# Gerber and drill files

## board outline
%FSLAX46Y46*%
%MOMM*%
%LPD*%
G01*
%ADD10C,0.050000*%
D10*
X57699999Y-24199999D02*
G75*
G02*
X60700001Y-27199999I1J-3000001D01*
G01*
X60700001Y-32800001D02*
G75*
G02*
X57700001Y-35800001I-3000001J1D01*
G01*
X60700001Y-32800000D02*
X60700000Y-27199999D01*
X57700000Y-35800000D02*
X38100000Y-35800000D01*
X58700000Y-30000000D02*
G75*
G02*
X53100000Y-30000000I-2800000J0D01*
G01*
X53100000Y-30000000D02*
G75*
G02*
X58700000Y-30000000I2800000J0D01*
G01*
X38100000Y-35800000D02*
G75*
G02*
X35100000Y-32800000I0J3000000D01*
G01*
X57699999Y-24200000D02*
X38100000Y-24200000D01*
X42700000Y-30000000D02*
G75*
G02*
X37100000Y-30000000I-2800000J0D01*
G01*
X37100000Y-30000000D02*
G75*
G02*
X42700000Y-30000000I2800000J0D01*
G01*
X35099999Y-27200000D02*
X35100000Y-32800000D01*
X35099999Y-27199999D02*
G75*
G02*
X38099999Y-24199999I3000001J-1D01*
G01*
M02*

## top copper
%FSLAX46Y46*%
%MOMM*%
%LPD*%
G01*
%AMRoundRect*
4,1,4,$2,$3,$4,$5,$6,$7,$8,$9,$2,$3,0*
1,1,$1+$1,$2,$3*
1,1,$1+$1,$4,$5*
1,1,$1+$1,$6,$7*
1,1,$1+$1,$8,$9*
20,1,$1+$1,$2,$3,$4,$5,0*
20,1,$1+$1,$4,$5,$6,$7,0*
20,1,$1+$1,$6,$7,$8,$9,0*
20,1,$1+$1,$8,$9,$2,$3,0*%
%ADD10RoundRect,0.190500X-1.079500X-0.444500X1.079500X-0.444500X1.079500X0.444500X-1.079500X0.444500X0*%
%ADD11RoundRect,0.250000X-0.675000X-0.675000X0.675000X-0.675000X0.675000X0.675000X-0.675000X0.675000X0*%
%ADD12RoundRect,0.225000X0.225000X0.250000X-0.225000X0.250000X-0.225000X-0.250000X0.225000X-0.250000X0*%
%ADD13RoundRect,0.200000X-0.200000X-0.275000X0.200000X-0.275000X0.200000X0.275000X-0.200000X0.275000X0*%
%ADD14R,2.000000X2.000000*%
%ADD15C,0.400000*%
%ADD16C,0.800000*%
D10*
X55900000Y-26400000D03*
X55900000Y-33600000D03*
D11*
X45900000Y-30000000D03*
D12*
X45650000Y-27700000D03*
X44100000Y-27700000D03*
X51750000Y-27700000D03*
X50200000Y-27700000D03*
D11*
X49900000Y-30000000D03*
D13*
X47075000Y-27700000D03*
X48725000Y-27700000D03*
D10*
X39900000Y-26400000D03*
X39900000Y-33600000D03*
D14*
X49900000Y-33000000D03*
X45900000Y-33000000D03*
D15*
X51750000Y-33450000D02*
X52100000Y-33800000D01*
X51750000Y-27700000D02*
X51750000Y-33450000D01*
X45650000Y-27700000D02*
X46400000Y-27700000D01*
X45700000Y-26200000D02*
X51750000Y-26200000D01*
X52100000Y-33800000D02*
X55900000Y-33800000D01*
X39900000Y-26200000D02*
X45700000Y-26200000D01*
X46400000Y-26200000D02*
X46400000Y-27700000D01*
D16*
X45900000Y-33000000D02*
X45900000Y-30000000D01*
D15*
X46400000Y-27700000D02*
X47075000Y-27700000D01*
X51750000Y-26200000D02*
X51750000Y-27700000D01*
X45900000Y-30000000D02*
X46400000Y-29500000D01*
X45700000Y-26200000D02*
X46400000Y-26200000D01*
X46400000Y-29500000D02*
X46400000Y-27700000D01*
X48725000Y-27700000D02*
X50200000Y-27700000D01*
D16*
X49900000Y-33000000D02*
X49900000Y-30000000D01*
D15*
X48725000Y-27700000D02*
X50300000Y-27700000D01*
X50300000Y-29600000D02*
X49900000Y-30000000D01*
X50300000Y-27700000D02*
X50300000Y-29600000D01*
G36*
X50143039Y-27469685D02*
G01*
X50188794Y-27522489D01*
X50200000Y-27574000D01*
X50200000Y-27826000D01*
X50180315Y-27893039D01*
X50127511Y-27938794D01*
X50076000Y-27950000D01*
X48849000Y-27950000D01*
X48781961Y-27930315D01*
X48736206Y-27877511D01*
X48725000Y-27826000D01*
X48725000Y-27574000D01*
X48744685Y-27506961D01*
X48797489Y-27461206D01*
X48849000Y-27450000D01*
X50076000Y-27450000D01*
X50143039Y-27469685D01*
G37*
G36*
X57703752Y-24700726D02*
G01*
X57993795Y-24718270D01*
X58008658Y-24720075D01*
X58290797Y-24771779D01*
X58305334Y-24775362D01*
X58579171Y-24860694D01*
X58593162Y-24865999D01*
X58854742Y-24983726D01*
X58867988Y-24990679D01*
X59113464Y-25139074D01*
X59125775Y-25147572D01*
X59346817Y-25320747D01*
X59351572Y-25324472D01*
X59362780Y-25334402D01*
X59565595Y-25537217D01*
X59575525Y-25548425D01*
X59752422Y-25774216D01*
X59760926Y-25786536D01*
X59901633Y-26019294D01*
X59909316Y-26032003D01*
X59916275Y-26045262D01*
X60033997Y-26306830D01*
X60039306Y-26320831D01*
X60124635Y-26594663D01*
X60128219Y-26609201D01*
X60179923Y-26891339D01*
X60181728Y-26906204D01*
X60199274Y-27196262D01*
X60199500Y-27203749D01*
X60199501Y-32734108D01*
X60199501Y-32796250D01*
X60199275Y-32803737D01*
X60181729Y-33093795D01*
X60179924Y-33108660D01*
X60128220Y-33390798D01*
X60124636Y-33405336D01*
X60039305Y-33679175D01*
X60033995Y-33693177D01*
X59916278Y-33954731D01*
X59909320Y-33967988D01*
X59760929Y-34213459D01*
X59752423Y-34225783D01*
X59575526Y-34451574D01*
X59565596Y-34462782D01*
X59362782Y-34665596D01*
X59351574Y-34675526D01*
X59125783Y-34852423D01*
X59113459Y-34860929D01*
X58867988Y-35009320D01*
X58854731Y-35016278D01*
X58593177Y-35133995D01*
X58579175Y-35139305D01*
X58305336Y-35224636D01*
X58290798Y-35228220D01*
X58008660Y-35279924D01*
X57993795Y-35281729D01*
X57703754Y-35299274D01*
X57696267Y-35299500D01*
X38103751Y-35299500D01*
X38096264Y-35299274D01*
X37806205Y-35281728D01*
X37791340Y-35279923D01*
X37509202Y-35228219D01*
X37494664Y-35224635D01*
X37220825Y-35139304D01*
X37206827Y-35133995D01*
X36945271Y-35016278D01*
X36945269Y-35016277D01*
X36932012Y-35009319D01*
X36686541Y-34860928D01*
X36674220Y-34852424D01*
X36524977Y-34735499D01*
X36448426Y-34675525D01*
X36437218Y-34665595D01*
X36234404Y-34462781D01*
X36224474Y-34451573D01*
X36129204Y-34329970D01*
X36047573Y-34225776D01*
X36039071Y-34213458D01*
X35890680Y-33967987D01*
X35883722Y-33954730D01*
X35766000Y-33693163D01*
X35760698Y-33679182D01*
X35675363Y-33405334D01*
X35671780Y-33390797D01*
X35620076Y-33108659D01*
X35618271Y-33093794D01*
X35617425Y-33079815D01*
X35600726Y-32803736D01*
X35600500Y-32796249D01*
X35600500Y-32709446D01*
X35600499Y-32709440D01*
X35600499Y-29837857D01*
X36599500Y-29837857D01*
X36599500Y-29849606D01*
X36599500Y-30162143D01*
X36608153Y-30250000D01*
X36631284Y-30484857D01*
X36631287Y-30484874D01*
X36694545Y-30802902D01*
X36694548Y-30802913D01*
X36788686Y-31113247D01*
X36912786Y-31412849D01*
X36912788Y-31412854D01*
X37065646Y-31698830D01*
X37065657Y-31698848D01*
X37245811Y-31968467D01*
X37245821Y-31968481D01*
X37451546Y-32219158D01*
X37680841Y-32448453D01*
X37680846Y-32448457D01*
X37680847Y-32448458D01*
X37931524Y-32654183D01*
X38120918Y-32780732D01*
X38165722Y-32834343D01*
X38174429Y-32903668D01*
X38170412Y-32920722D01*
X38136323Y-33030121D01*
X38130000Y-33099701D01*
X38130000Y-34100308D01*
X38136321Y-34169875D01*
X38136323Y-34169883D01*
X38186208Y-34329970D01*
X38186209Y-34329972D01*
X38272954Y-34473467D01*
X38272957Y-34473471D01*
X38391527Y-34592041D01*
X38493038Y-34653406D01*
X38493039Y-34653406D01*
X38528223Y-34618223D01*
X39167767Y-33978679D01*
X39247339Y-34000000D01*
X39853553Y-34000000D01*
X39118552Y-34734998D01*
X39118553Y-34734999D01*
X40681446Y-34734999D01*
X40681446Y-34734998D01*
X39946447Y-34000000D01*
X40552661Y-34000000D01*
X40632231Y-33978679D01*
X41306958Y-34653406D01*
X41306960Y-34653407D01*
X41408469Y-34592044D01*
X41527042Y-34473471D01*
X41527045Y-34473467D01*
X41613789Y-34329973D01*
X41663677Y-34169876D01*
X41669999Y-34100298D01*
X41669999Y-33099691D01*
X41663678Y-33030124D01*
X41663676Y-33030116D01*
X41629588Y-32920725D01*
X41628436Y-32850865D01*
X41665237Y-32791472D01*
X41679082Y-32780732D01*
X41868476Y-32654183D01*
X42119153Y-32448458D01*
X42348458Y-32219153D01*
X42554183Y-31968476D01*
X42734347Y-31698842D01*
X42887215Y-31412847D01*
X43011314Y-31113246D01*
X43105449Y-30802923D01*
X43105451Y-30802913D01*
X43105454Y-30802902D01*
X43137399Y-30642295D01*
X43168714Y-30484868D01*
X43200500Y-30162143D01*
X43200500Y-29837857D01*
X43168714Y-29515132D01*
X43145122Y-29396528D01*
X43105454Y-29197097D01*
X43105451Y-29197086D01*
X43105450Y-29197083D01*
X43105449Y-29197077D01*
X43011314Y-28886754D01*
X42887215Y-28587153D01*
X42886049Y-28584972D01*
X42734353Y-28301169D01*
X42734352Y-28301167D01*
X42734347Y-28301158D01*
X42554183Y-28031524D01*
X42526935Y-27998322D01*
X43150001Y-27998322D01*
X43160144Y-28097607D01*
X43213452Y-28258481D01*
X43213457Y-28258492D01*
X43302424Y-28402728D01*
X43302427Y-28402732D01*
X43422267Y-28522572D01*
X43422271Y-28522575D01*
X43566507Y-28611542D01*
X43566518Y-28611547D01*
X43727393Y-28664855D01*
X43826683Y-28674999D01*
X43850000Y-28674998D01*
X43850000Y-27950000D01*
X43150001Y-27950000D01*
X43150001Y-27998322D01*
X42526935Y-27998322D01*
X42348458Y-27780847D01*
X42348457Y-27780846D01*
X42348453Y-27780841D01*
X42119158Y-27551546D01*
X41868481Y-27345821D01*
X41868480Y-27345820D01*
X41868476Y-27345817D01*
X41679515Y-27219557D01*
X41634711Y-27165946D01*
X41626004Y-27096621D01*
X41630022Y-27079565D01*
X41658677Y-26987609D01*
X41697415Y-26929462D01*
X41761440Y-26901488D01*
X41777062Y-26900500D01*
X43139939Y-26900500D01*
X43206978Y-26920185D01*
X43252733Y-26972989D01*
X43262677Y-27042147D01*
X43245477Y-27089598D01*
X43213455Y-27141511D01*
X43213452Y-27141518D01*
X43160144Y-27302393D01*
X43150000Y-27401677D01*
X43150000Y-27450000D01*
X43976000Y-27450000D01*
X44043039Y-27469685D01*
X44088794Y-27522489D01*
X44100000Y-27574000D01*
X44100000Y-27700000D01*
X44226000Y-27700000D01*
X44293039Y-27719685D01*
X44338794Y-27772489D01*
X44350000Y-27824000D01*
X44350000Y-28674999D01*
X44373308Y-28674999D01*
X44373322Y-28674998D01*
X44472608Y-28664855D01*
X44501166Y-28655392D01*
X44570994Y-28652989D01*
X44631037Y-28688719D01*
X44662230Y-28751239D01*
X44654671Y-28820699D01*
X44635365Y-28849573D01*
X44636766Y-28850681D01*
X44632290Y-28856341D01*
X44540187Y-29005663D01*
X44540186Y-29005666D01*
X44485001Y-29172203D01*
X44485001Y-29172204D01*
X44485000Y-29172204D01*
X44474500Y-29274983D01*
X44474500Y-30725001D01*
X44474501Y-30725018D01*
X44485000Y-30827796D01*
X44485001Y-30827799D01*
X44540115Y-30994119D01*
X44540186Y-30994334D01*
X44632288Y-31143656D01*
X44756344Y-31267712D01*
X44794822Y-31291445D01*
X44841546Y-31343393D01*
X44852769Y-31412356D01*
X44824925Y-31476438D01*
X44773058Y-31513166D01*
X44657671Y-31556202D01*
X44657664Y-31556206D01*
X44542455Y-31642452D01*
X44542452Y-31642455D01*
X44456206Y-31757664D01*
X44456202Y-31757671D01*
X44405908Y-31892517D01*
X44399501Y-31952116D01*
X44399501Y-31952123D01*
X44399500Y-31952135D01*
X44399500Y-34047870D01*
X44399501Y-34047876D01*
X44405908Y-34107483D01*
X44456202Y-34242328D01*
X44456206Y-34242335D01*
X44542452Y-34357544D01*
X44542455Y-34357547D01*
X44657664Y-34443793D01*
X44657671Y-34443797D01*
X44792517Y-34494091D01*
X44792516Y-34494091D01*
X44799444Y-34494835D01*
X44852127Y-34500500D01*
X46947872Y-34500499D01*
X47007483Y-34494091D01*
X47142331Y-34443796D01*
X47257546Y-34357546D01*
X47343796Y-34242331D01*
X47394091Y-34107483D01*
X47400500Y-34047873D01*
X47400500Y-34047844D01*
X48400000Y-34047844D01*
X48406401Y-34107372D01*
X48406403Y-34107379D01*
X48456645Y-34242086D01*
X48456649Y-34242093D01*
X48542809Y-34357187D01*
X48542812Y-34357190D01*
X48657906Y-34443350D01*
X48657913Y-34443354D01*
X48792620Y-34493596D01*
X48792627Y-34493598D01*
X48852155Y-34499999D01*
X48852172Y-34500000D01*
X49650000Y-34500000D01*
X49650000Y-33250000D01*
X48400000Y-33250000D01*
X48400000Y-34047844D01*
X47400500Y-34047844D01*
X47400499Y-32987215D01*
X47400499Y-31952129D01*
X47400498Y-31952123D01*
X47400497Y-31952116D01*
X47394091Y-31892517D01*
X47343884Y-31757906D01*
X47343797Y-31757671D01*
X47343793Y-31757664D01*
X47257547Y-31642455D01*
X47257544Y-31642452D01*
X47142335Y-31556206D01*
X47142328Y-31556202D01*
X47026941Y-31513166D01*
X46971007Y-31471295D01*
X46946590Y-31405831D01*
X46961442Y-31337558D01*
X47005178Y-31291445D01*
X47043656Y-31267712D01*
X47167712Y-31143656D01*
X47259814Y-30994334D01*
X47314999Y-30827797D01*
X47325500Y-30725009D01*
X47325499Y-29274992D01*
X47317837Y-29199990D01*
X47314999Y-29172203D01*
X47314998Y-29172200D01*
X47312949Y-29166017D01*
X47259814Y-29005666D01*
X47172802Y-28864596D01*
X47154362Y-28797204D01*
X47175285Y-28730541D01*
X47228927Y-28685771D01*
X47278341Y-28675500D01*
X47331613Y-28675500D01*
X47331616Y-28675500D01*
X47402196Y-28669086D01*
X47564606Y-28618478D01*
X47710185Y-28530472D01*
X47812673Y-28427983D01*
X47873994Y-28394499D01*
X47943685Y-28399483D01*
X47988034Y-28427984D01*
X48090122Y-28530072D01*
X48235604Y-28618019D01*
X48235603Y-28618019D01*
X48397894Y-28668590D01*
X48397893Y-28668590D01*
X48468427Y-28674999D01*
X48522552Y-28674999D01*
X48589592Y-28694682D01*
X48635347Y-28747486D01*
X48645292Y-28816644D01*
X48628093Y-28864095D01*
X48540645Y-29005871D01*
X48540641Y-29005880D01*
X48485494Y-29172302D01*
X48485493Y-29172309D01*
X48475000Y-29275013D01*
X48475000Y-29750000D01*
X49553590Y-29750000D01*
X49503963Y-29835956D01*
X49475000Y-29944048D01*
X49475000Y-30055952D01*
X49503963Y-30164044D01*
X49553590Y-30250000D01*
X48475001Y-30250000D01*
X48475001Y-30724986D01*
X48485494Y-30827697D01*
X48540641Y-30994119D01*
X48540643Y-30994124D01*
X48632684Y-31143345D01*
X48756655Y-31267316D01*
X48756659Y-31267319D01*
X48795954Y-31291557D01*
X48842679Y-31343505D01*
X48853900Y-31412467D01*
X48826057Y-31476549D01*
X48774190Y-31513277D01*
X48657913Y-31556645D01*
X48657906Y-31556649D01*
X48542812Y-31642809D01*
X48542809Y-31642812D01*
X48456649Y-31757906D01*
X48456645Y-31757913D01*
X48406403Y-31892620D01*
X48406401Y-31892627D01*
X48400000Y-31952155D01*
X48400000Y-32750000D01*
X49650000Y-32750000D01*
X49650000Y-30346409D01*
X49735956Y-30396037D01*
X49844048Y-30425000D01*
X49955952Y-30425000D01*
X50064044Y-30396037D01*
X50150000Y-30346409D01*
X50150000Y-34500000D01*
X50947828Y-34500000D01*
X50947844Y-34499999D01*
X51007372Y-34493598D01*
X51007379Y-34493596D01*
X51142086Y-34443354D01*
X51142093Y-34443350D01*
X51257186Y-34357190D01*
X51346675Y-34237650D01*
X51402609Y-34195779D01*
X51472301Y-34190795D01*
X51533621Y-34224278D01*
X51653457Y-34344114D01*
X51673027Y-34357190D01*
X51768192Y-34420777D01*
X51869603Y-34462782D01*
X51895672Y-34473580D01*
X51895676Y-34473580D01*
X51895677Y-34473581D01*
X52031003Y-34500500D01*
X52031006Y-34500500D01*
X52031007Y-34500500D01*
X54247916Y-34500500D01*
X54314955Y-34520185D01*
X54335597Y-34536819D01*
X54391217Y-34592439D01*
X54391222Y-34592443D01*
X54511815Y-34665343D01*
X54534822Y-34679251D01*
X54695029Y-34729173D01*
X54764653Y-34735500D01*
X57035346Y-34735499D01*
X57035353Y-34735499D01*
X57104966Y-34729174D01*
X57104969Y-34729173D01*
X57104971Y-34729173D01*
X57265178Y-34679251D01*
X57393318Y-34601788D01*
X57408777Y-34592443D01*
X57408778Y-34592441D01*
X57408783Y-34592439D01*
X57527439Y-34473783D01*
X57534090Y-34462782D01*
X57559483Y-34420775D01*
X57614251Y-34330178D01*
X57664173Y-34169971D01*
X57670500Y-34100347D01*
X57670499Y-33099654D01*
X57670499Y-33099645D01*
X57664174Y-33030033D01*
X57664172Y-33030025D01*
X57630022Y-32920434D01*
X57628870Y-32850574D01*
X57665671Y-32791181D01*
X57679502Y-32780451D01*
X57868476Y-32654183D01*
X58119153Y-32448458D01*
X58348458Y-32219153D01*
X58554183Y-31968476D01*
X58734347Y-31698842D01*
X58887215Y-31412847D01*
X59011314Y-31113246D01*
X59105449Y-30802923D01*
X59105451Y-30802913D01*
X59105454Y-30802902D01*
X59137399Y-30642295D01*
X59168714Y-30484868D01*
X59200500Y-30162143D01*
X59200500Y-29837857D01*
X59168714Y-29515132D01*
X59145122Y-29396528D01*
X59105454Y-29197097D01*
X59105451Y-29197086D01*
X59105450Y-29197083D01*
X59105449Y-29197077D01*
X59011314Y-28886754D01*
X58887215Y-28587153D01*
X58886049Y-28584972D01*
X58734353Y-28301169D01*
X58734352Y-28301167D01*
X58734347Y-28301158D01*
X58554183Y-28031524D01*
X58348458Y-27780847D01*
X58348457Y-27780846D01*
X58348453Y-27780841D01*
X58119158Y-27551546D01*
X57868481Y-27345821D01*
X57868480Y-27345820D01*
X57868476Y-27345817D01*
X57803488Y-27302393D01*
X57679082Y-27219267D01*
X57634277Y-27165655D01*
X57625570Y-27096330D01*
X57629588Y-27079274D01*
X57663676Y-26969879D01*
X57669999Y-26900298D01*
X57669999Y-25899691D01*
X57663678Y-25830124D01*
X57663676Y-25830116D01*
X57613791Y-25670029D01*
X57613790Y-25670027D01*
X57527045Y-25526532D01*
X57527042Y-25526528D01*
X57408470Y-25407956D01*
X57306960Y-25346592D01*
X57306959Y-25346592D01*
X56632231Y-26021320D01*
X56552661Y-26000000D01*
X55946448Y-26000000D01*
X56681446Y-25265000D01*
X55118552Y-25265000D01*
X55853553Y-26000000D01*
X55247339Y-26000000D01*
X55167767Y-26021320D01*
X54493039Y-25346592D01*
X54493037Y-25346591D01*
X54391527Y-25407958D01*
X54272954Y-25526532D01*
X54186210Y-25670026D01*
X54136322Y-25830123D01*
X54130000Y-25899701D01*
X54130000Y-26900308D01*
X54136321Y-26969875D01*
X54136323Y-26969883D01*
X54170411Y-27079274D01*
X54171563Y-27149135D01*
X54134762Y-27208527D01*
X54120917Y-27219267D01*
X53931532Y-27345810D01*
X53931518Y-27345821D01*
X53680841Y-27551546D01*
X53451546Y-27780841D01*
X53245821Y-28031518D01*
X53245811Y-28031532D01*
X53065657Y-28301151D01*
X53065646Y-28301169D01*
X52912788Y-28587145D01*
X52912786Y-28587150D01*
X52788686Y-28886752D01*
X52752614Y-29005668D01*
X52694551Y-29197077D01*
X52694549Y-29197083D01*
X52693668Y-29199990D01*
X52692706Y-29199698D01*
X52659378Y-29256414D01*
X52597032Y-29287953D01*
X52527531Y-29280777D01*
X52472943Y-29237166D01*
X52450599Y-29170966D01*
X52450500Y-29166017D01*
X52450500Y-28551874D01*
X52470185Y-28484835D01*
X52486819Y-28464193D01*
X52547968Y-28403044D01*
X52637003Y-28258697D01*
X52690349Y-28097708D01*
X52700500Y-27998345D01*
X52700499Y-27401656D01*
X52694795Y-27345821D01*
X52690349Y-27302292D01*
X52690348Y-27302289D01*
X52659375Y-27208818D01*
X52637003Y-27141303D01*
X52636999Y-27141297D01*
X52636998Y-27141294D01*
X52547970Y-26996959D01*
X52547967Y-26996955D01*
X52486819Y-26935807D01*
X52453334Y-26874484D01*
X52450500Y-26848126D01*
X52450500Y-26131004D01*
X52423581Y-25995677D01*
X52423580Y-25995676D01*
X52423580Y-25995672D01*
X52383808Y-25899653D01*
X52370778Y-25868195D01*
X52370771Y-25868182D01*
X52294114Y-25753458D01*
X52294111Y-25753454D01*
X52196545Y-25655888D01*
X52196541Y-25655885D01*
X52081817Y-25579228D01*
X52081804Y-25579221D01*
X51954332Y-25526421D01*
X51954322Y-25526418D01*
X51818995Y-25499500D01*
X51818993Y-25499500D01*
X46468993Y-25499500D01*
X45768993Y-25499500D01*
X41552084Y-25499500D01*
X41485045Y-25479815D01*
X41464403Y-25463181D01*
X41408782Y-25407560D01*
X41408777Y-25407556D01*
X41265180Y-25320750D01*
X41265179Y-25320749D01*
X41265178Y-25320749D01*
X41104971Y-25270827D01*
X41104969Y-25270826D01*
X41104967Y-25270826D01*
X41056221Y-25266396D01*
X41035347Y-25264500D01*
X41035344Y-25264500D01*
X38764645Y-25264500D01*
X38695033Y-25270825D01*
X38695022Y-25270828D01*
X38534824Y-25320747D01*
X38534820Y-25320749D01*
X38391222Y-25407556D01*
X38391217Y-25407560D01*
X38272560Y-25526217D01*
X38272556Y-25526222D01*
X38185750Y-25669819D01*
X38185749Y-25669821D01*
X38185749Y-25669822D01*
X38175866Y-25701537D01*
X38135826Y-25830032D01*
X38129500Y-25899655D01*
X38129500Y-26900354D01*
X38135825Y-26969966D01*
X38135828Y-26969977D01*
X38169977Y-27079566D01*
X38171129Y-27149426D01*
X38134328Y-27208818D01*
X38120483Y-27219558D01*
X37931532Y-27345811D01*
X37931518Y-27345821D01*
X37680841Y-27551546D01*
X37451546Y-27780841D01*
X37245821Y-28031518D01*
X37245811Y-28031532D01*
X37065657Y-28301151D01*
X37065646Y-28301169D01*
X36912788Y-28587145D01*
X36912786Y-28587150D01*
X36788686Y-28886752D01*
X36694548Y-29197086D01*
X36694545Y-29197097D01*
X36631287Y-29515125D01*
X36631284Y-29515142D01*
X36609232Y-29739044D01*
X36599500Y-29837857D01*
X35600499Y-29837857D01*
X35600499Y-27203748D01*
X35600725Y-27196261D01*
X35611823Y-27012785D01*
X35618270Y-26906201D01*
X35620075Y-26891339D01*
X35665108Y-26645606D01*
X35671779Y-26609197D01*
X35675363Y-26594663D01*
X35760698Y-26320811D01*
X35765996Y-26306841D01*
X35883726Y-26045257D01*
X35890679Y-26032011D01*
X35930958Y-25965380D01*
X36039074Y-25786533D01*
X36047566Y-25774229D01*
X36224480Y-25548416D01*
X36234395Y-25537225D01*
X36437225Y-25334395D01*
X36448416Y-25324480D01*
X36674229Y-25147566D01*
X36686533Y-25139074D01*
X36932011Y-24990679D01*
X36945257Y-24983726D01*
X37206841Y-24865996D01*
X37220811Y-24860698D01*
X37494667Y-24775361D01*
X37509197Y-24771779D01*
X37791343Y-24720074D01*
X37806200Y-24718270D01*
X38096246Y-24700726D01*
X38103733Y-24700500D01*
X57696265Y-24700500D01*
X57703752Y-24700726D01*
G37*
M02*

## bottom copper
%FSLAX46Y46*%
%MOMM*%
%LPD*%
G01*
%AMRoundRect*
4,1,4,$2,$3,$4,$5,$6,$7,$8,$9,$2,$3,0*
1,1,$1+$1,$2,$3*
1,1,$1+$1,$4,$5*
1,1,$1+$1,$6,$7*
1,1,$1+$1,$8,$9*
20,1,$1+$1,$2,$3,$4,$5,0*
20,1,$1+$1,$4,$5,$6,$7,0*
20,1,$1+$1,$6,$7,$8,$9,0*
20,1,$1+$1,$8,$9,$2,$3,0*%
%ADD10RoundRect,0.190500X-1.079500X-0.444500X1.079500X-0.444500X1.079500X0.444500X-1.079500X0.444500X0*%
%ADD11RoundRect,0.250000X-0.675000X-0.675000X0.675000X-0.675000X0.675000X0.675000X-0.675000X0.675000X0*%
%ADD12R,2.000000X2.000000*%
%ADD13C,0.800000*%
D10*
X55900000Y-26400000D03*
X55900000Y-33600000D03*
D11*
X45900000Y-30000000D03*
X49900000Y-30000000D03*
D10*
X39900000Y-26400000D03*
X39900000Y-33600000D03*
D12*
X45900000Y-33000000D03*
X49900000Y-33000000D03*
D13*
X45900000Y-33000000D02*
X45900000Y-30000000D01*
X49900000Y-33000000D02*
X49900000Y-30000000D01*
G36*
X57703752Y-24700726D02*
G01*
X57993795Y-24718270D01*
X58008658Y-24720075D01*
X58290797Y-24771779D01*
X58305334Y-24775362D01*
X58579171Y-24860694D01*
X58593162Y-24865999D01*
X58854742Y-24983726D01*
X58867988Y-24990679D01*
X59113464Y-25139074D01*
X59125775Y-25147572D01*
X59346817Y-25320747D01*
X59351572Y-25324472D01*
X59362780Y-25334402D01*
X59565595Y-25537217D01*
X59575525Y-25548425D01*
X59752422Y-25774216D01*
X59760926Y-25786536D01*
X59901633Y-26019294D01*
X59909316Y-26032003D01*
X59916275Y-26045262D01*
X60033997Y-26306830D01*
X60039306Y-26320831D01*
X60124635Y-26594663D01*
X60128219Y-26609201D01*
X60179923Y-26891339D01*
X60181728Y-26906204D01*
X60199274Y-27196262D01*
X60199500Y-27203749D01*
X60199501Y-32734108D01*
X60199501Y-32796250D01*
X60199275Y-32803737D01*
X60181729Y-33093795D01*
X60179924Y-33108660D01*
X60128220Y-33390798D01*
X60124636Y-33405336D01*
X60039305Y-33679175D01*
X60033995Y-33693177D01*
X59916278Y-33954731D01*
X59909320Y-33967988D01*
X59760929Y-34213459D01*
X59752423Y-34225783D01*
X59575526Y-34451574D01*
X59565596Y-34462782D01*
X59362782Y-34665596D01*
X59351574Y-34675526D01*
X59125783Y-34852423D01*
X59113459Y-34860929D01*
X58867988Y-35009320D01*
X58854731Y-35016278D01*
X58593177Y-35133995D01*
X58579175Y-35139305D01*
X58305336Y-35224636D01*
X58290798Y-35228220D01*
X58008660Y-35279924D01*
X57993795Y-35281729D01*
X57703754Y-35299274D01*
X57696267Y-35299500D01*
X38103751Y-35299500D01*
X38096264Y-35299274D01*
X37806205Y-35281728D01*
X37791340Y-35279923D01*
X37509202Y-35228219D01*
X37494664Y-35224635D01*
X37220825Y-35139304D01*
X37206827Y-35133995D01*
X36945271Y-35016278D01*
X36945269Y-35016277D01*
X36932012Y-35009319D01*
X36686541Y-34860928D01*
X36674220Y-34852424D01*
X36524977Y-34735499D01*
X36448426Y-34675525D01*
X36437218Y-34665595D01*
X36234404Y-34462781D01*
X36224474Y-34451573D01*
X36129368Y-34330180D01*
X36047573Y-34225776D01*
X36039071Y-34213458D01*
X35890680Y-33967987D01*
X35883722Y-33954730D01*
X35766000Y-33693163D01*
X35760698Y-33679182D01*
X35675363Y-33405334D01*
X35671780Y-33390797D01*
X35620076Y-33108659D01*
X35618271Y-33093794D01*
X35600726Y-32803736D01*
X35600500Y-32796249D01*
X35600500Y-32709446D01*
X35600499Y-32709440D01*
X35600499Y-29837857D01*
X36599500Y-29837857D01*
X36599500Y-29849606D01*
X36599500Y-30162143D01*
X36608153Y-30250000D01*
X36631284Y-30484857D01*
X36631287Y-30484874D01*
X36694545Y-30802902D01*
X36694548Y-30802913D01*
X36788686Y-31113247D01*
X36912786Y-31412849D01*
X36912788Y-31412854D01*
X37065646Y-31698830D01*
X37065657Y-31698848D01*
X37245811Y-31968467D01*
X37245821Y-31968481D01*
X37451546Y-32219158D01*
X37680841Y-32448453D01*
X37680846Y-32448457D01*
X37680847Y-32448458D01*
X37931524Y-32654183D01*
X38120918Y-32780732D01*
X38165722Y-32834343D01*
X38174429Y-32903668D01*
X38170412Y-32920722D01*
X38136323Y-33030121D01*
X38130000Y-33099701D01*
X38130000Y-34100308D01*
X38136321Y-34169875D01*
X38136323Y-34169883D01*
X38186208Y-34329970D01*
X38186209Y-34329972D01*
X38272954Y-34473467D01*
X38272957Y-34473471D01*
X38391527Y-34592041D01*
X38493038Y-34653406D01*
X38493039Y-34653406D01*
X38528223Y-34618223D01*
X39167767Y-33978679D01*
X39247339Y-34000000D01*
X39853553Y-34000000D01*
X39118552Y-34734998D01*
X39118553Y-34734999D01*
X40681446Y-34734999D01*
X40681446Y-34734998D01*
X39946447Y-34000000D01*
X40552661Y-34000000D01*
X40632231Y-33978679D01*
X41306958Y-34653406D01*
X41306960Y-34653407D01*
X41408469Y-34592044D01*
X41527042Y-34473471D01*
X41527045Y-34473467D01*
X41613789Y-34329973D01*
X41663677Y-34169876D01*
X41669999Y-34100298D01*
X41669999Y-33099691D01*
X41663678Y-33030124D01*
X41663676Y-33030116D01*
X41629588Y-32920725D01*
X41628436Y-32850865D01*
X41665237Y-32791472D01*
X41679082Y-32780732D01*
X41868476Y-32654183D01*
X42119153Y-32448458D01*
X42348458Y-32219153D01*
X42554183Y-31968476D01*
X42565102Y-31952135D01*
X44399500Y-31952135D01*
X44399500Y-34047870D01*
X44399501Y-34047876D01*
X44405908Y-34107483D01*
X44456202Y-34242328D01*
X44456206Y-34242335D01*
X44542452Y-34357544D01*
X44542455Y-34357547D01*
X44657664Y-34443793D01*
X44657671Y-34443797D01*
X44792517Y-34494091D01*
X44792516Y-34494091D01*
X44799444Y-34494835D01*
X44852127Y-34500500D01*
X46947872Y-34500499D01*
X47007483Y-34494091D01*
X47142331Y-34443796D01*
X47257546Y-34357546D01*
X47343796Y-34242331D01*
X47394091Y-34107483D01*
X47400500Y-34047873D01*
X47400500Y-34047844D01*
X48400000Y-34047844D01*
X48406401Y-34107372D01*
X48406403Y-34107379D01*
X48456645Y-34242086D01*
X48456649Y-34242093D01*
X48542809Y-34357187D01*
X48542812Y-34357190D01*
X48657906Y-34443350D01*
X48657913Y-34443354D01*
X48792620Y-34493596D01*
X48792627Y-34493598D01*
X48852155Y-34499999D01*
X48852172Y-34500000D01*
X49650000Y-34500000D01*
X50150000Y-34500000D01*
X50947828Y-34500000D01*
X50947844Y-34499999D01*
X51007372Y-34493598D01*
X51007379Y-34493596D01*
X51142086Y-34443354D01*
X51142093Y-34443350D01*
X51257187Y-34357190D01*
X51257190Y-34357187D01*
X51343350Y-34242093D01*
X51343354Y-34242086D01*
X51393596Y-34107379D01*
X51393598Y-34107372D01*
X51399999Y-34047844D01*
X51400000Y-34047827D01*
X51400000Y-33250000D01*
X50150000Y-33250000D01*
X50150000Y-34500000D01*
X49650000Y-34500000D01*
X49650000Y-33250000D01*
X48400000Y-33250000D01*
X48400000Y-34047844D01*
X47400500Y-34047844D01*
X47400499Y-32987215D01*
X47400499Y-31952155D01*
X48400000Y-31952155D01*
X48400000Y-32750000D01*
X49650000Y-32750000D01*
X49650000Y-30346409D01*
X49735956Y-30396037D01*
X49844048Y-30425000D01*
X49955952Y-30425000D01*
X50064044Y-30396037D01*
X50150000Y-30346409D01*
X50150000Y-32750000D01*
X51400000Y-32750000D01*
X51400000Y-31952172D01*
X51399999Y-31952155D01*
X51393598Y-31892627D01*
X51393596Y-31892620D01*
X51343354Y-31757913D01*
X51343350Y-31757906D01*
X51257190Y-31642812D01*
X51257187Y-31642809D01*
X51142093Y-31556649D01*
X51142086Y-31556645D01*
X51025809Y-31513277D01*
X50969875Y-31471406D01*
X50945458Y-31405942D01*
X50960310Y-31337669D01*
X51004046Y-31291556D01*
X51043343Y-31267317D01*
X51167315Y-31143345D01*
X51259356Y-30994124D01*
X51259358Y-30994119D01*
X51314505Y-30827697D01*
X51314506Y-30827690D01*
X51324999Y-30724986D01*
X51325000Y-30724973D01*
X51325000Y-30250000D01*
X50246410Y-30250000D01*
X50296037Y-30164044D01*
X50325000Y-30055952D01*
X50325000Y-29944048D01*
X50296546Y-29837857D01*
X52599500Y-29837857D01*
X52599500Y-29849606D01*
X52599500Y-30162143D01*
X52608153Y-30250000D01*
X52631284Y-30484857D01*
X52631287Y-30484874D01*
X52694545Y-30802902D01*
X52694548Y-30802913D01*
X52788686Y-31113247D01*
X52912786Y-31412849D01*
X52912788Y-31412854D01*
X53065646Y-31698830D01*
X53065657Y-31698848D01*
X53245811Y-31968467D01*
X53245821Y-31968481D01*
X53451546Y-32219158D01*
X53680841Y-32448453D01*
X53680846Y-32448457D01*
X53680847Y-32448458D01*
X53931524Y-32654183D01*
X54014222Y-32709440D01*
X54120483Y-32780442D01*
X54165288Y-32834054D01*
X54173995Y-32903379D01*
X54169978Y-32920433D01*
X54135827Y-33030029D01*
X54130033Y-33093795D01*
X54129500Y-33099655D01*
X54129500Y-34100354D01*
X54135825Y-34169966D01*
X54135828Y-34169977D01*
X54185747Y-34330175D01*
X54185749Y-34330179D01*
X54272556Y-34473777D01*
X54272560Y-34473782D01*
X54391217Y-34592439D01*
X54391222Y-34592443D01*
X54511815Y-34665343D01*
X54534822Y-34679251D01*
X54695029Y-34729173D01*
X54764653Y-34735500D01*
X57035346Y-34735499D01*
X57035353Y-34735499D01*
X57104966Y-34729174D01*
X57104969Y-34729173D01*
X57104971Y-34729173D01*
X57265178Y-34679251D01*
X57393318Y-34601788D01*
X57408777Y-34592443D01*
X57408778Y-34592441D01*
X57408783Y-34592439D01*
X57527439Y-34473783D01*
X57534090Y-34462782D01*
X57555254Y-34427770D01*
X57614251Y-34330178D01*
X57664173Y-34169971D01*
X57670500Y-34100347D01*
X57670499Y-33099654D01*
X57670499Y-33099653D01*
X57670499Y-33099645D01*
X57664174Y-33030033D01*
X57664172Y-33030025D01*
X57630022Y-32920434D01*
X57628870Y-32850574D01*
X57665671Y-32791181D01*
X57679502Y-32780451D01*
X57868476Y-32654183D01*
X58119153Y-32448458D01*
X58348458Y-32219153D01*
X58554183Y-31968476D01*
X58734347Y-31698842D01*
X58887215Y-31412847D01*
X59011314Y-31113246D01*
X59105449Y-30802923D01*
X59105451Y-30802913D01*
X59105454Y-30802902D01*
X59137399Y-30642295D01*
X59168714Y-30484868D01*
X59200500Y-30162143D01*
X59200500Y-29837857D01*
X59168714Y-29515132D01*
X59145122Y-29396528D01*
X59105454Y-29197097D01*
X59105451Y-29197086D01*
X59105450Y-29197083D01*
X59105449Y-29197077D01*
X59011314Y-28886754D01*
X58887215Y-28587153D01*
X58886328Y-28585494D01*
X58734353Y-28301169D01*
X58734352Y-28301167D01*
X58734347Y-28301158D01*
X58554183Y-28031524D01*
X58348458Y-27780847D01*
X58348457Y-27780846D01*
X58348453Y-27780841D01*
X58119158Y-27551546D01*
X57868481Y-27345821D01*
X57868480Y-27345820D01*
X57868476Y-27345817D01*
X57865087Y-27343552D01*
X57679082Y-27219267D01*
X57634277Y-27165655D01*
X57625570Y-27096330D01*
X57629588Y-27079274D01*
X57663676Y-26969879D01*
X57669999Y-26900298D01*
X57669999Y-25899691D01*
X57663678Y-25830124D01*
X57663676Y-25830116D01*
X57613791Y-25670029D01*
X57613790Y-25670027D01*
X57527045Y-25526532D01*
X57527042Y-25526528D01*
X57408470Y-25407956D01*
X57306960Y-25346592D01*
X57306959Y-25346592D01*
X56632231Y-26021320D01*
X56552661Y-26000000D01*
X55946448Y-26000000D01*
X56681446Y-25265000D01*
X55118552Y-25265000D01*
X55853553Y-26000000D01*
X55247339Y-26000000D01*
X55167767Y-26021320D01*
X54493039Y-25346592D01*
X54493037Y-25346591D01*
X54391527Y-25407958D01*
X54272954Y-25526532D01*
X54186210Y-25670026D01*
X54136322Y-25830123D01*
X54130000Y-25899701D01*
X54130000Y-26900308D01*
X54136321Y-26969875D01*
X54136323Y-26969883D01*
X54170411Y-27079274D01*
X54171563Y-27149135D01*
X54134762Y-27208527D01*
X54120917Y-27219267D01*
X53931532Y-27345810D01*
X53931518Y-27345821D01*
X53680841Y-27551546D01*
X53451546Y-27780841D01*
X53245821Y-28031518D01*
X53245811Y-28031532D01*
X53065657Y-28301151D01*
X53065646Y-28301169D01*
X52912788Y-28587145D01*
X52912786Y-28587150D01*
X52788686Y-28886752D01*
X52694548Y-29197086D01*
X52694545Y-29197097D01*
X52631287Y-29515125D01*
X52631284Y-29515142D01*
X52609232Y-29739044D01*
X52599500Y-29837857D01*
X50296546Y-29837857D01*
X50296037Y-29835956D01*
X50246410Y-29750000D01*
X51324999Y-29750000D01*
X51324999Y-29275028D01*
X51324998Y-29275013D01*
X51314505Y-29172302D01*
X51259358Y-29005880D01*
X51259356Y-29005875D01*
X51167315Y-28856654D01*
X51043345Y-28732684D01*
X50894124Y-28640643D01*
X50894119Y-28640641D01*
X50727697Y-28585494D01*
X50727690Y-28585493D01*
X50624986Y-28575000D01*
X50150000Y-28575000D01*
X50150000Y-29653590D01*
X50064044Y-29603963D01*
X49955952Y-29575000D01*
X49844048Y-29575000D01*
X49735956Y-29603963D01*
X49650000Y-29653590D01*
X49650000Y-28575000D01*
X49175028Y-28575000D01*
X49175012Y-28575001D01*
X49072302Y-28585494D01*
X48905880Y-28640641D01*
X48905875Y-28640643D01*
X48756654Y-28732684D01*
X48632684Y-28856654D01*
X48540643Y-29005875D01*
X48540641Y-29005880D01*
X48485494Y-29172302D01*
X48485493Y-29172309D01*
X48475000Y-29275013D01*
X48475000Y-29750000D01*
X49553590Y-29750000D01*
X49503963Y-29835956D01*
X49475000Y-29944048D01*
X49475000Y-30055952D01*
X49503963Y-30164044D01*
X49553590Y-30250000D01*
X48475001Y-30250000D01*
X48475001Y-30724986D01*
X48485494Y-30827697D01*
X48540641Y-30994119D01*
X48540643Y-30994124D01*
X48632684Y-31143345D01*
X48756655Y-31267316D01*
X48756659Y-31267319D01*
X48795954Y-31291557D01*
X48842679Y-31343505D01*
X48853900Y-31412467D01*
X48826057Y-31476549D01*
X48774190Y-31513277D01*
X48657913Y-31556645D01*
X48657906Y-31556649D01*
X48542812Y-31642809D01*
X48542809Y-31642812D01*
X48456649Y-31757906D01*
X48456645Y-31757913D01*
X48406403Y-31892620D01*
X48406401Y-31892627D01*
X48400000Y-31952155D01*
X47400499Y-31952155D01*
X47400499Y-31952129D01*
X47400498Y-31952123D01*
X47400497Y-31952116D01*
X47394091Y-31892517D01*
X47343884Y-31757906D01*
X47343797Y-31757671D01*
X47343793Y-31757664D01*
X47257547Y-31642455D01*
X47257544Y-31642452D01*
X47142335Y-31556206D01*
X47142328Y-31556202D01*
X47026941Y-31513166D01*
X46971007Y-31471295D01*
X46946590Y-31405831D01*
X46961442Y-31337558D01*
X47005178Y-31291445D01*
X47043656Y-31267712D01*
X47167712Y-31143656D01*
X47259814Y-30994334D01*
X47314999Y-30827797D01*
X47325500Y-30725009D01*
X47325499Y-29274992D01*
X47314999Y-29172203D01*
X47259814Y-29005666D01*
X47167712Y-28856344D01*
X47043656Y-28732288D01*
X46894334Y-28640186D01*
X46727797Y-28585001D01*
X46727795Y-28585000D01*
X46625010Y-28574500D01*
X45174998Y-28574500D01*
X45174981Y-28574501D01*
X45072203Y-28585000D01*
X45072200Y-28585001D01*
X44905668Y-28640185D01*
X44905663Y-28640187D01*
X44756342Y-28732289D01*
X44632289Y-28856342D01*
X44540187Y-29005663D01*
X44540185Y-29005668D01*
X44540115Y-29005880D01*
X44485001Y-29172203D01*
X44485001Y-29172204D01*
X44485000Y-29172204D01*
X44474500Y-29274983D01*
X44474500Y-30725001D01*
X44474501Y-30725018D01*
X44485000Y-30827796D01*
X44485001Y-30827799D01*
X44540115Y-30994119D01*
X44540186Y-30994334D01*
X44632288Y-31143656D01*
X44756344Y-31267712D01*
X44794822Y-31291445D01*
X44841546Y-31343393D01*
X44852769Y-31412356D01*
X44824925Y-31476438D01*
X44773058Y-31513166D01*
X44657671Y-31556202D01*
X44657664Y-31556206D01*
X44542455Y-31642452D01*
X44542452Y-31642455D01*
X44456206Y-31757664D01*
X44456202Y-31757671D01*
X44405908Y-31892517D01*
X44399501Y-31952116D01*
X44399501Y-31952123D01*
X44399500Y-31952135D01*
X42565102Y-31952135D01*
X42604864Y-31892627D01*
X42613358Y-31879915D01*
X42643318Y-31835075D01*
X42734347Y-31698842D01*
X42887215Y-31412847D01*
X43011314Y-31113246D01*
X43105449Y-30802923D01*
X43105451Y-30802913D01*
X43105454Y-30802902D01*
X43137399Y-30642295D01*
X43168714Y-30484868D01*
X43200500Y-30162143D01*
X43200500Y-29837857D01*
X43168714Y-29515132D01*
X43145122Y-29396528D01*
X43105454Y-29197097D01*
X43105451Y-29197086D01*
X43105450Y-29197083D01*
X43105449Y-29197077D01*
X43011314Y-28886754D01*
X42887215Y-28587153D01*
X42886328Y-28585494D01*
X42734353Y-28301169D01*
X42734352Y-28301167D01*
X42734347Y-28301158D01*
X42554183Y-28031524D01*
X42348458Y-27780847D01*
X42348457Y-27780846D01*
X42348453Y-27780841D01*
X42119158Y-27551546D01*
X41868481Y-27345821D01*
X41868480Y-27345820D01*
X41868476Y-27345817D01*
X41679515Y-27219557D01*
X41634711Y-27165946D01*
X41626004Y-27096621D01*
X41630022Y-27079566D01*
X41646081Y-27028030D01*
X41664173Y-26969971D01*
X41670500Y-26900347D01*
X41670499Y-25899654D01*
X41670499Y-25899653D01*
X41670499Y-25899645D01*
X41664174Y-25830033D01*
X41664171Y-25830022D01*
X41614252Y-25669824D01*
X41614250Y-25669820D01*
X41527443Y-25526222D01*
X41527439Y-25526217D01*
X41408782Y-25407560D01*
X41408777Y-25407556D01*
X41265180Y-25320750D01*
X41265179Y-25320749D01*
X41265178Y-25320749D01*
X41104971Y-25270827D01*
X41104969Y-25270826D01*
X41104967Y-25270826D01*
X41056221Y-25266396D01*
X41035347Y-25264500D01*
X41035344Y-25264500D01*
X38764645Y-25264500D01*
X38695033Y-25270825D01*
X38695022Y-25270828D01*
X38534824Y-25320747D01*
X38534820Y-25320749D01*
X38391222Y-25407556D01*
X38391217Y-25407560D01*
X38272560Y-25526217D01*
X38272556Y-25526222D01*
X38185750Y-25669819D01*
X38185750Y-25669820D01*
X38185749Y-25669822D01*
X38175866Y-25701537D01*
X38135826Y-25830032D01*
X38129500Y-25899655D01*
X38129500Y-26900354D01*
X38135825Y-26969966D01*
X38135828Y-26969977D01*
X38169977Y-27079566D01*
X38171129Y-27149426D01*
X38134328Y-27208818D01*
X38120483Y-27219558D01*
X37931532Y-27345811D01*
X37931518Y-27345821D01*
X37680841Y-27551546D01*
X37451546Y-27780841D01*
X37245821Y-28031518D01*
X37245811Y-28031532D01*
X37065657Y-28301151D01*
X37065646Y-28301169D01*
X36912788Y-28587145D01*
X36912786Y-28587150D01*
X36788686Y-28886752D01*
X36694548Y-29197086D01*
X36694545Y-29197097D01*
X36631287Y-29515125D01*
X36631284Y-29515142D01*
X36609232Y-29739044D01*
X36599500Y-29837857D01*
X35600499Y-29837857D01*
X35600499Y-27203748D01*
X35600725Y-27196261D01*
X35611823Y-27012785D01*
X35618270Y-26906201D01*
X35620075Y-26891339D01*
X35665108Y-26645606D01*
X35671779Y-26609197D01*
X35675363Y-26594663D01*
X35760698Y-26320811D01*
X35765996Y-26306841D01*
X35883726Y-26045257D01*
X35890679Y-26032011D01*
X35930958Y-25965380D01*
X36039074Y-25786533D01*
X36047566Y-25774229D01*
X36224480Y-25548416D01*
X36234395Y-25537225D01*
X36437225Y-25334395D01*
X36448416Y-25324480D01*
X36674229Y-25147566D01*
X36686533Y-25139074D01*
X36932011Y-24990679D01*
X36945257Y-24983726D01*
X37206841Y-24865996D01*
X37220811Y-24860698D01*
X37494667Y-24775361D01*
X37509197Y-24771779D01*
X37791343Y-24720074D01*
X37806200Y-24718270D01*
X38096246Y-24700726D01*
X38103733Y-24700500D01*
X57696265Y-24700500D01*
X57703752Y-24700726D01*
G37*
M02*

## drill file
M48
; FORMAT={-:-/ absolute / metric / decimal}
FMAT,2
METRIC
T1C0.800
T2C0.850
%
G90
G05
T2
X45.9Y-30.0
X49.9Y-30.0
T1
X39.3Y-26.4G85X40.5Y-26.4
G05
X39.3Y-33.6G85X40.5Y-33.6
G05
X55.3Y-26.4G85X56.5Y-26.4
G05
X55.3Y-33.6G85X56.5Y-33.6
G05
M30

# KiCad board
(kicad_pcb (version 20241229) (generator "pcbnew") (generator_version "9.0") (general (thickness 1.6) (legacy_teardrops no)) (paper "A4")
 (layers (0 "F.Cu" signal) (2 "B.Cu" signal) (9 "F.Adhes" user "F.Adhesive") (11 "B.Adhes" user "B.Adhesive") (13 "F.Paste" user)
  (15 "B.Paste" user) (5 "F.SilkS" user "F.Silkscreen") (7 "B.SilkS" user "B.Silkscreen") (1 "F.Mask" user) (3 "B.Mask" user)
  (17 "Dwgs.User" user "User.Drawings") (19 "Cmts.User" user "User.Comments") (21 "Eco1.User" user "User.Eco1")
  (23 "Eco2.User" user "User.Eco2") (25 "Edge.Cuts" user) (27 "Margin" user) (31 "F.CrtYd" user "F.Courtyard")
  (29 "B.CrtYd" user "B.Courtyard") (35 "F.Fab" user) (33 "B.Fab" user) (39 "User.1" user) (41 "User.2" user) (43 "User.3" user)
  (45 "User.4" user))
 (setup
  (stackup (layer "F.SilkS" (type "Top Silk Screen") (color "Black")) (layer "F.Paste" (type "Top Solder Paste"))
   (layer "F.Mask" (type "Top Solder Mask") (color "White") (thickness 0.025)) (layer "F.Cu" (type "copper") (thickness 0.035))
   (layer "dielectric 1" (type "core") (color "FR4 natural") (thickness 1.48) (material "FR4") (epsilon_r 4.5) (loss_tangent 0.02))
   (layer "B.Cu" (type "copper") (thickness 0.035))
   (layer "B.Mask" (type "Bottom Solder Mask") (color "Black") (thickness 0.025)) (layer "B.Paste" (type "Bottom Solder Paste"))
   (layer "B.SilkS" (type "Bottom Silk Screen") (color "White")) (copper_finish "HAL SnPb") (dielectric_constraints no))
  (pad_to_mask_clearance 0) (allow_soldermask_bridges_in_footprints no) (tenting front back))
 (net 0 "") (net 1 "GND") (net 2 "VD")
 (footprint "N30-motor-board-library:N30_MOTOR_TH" (layer "F.Cu") (at 55.9 30)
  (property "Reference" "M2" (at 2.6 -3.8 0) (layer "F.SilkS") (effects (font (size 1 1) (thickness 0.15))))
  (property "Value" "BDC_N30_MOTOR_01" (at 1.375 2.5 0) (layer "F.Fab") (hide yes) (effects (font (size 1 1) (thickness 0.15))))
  (pad "1" thru_hole roundrect (at 0 -3.6) (size 2.54 1.27) (drill oval 2 0.8) (layers "*.Cu" "*.Mask") (remove_unused_layers no)
   (roundrect_rratio 0.15) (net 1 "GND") (thermal_bridge_angle 45))
  (pad "2" thru_hole roundrect (at 0 3.6) (size 2.54 1.27) (drill oval 2 0.8) (layers "*.Cu" "*.Mask") (remove_unused_layers no)
   (roundrect_rratio 0.15) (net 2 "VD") (thermal_bridge_angle 45)))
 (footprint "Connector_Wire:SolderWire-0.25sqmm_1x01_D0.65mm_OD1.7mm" (layer "F.Cu") (at 45.9 30)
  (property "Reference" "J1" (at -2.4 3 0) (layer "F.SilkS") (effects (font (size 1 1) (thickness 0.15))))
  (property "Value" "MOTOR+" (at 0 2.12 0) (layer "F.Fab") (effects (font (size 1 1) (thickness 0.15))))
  (pad "1" thru_hole roundrect (at 0 0) (size 1.85 1.85) (drill 0.85) (layers "*.Cu" "*.Mask") (remove_unused_layers no)
   (roundrect_rratio 0.135135) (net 2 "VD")))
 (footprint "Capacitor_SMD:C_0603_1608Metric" (layer "F.Cu") (at 44.875 27.7 180)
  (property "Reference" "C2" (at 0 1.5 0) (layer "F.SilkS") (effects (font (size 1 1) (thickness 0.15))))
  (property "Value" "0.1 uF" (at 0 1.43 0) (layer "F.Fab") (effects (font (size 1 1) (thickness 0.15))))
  (pad "1" smd roundrect (at -0.775 0 180) (size 0.9 0.95) (layers "F.Cu" "F.Mask" "F.Paste") (roundrect_rratio 0.25) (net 2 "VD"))
  (pad "2" smd roundrect (at 0.775 0 180) (size 0.9 0.95) (layers "F.Cu" "F.Mask" "F.Paste") (roundrect_rratio 0.25) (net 1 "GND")))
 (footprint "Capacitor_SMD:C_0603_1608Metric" (layer "F.Cu") (at 50.975 27.7 180)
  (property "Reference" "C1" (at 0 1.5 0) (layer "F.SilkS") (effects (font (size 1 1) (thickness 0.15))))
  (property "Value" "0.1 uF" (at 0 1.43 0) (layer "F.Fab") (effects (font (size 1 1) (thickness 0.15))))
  (pad "1" smd roundrect (at -0.775 0 180) (size 0.9 0.95) (layers "F.Cu" "F.Mask" "F.Paste") (roundrect_rratio 0.25) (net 2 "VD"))
  (pad "2" smd roundrect (at 0.775 0 180) (size 0.9 0.95) (layers "F.Cu" "F.Mask" "F.Paste") (roundrect_rratio 0.25) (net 1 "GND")))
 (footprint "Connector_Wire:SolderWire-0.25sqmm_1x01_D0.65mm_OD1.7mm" (layer "F.Cu") (at 49.9 30)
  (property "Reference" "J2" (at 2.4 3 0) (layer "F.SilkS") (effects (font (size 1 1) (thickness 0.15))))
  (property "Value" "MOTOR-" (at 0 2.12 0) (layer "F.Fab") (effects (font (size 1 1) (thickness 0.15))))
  (pad "1" thru_hole roundrect (at 0 0) (size 1.85 1.85) (drill 0.85) (layers "*.Cu" "*.Mask") (remove_unused_layers no)
   (roundrect_rratio 0.135135) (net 1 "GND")))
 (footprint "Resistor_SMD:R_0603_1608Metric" (layer "F.Cu") (at 47.9 27.7)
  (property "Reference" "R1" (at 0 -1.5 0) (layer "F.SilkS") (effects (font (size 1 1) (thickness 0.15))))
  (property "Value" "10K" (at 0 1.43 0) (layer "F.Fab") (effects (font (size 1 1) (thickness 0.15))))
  (pad "1" smd roundrect (at -0.825 0) (size 0.8 0.95) (layers "F.Cu" "F.Mask" "F.Paste") (roundrect_rratio 0.25) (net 2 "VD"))
  (pad "2" smd roundrect (at 0.825 0) (size 0.8 0.95) (layers "F.Cu" "F.Mask" "F.Paste") (roundrect_rratio 0.25) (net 1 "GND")))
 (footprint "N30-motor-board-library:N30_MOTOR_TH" (layer "F.Cu") (at 39.9 30)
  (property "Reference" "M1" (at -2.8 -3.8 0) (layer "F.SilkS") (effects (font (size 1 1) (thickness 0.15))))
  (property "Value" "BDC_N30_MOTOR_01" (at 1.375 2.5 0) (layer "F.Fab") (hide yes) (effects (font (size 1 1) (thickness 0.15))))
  (pad "1" thru_hole roundrect (at 0 -3.6) (size 2.54 1.27) (drill oval 2 0.8) (layers "*.Cu" "*.Mask") (remove_unused_layers no)
   (roundrect_rratio 0.15) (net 2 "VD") (thermal_bridge_angle 45))
  (pad "2" thru_hole roundrect (at 0 3.6) (size 2.54 1.27) (drill oval 2 0.8) (layers "*.Cu" "*.Mask") (remove_unused_layers no)
   (roundrect_rratio 0.15) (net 1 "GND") (thermal_bridge_angle 45)))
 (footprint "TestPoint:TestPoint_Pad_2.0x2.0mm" (layer "F.Cu") (at 49.9 33)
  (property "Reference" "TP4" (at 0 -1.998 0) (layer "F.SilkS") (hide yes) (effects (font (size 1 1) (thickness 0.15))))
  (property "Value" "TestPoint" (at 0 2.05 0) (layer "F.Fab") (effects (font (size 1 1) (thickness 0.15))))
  (pad "1" smd rect (at 0 0) (size 2 2) (layers "F.Cu" "F.Mask") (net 1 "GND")))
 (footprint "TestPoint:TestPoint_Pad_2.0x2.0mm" (layer "F.Cu") (at 45.9 33)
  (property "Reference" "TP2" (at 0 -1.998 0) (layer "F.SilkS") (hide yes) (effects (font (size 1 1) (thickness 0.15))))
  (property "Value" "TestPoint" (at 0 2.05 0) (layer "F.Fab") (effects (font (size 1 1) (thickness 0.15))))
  (pad "1" smd rect (at 0 0) (size 2 2) (layers "F.Cu" "F.Mask") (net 2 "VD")))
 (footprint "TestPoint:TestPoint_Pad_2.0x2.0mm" (layer "B.Cu") (at 45.9 33)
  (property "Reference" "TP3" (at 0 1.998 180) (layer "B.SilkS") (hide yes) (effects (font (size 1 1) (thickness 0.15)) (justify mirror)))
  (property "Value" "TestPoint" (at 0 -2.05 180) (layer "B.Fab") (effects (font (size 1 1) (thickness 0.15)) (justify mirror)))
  (pad "1" smd rect (at 0 0) (size 2 2) (layers "B.Cu" "B.Mask") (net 2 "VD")))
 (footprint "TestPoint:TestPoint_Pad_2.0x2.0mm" (layer "B.Cu") (at 49.9 33)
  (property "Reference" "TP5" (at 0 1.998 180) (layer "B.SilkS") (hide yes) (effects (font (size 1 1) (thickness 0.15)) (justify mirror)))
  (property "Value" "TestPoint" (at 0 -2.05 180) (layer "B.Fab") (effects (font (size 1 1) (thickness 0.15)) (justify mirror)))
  (pad "1" smd rect (at 0 0) (size 2 2) (layers "B.Cu" "B.Mask") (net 1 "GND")))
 (gr_arc (start 57.699999 24.199999) (mid 59.82132 25.078679) (end 60.7 27.199999) (stroke (width 0.05) (type default)) (layer "Edge.Cuts"))
 (gr_arc (start 60.700001 32.800001) (mid 59.821321 34.921321) (end 57.700001 35.800001) (stroke (width 0.05) (type default))
  (layer "Edge.Cuts"))
 (gr_line (start 60.700001 32.8) (end 60.7 27.199999) (stroke (width 0.05) (type default)) (layer "Edge.Cuts"))
 (gr_line (start 57.7 35.8) (end 38.1 35.8) (stroke (width 0.05) (type default)) (layer "Edge.Cuts"))
 (gr_circle (center 55.9 30) (end 58.7 30) (stroke (width 0.05) (type solid)) (fill no) (layer "Edge.Cuts"))
 (gr_arc (start 38.1 35.8) (mid 35.97868 34.92132) (end 35.1 32.8) (stroke (width 0.05) (type default)) (layer "Edge.Cuts"))
 (gr_line (start 57.699999 24.2) (end 38.1 24.2) (stroke (width 0.05) (type default)) (layer "Edge.Cuts"))
 (gr_circle (center 39.9 30) (end 42.7 30) (stroke (width 0.05) (type solid)) (fill no) (layer "Edge.Cuts"))
 (gr_line (start 35.099999 27.2) (end 35.1 32.8) (stroke (width 0.05) (type default)) (layer "Edge.Cuts"))
 (gr_arc (start 35.099999 27.199999) (mid 35.978679 25.078679) (end 38.099999 24.199999) (stroke (width 0.05) (type default))
  (layer "Edge.Cuts"))
 (segment (start 51.75 33.45) (end 52.1 33.8) (width 0.4) (layer "F.Cu") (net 2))
 (segment (start 51.75 27.7) (end 51.75 33.45) (width 0.4) (layer "F.Cu") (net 2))
 (segment (start 45.65 27.7) (end 46.4 27.7) (width 0.4) (layer "F.Cu") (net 2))
 (segment (start 45.7 26.2) (end 51.75 26.2) (width 0.4) (layer "F.Cu") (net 2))
 (segment (start 52.1 33.8) (end 55.9 33.8) (width 0.4) (layer "F.Cu") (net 2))
 (segment (start 39.9 26.2) (end 45.7 26.2) (width 0.4) (layer "F.Cu") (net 2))
 (segment (start 46.4 26.2) (end 46.4 27.7) (width 0.4) (layer "F.Cu") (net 2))
 (segment (start 45.9 33) (end 45.9 30) (width 0.8) (layer "F.Cu") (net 2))
 (segment (start 46.4 27.7) (end 47.075 27.7) (width 0.4) (layer "F.Cu") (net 2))
 (segment (start 51.75 26.2) (end 51.75 27.7) (width 0.4) (layer "F.Cu") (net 2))
 (segment (start 45.9 30) (end 46.4 29.5) (width 0.4) (layer "F.Cu") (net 2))
 (segment (start 45.7 26.2) (end 46.4 26.2) (width 0.4) (layer "F.Cu") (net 2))
 (segment (start 46.4 29.5) (end 46.4 27.7) (width 0.4) (layer "F.Cu") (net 2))
 (segment (start 45.9 33) (end 45.9 30) (width 0.8) (layer "B.Cu") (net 2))
 (segment (start 48.725 27.7) (end 50.2 27.7) (width 0.4) (layer "F.Cu") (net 1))
 (segment (start 49.9 33) (end 49.9 30) (width 0.8) (layer "F.Cu") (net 1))
 (segment (start 48.725 27.7) (end 50.3 27.7) (width 0.4) (layer "F.Cu") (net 1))
 (segment (start 50.3 29.6) (end 49.9 30) (width 0.4) (layer "F.Cu") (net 1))
 (segment (start 50.3 27.7) (end 50.3 29.6) (width 0.4) (layer "F.Cu") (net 1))
 (segment (start 49.9 33) (end 49.9 30) (width 0.8) (layer "B.Cu") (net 1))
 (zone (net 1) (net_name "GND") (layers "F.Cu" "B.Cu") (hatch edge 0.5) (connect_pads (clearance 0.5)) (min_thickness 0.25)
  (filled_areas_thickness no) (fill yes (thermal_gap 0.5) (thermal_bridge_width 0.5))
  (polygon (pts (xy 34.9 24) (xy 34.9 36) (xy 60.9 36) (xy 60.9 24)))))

